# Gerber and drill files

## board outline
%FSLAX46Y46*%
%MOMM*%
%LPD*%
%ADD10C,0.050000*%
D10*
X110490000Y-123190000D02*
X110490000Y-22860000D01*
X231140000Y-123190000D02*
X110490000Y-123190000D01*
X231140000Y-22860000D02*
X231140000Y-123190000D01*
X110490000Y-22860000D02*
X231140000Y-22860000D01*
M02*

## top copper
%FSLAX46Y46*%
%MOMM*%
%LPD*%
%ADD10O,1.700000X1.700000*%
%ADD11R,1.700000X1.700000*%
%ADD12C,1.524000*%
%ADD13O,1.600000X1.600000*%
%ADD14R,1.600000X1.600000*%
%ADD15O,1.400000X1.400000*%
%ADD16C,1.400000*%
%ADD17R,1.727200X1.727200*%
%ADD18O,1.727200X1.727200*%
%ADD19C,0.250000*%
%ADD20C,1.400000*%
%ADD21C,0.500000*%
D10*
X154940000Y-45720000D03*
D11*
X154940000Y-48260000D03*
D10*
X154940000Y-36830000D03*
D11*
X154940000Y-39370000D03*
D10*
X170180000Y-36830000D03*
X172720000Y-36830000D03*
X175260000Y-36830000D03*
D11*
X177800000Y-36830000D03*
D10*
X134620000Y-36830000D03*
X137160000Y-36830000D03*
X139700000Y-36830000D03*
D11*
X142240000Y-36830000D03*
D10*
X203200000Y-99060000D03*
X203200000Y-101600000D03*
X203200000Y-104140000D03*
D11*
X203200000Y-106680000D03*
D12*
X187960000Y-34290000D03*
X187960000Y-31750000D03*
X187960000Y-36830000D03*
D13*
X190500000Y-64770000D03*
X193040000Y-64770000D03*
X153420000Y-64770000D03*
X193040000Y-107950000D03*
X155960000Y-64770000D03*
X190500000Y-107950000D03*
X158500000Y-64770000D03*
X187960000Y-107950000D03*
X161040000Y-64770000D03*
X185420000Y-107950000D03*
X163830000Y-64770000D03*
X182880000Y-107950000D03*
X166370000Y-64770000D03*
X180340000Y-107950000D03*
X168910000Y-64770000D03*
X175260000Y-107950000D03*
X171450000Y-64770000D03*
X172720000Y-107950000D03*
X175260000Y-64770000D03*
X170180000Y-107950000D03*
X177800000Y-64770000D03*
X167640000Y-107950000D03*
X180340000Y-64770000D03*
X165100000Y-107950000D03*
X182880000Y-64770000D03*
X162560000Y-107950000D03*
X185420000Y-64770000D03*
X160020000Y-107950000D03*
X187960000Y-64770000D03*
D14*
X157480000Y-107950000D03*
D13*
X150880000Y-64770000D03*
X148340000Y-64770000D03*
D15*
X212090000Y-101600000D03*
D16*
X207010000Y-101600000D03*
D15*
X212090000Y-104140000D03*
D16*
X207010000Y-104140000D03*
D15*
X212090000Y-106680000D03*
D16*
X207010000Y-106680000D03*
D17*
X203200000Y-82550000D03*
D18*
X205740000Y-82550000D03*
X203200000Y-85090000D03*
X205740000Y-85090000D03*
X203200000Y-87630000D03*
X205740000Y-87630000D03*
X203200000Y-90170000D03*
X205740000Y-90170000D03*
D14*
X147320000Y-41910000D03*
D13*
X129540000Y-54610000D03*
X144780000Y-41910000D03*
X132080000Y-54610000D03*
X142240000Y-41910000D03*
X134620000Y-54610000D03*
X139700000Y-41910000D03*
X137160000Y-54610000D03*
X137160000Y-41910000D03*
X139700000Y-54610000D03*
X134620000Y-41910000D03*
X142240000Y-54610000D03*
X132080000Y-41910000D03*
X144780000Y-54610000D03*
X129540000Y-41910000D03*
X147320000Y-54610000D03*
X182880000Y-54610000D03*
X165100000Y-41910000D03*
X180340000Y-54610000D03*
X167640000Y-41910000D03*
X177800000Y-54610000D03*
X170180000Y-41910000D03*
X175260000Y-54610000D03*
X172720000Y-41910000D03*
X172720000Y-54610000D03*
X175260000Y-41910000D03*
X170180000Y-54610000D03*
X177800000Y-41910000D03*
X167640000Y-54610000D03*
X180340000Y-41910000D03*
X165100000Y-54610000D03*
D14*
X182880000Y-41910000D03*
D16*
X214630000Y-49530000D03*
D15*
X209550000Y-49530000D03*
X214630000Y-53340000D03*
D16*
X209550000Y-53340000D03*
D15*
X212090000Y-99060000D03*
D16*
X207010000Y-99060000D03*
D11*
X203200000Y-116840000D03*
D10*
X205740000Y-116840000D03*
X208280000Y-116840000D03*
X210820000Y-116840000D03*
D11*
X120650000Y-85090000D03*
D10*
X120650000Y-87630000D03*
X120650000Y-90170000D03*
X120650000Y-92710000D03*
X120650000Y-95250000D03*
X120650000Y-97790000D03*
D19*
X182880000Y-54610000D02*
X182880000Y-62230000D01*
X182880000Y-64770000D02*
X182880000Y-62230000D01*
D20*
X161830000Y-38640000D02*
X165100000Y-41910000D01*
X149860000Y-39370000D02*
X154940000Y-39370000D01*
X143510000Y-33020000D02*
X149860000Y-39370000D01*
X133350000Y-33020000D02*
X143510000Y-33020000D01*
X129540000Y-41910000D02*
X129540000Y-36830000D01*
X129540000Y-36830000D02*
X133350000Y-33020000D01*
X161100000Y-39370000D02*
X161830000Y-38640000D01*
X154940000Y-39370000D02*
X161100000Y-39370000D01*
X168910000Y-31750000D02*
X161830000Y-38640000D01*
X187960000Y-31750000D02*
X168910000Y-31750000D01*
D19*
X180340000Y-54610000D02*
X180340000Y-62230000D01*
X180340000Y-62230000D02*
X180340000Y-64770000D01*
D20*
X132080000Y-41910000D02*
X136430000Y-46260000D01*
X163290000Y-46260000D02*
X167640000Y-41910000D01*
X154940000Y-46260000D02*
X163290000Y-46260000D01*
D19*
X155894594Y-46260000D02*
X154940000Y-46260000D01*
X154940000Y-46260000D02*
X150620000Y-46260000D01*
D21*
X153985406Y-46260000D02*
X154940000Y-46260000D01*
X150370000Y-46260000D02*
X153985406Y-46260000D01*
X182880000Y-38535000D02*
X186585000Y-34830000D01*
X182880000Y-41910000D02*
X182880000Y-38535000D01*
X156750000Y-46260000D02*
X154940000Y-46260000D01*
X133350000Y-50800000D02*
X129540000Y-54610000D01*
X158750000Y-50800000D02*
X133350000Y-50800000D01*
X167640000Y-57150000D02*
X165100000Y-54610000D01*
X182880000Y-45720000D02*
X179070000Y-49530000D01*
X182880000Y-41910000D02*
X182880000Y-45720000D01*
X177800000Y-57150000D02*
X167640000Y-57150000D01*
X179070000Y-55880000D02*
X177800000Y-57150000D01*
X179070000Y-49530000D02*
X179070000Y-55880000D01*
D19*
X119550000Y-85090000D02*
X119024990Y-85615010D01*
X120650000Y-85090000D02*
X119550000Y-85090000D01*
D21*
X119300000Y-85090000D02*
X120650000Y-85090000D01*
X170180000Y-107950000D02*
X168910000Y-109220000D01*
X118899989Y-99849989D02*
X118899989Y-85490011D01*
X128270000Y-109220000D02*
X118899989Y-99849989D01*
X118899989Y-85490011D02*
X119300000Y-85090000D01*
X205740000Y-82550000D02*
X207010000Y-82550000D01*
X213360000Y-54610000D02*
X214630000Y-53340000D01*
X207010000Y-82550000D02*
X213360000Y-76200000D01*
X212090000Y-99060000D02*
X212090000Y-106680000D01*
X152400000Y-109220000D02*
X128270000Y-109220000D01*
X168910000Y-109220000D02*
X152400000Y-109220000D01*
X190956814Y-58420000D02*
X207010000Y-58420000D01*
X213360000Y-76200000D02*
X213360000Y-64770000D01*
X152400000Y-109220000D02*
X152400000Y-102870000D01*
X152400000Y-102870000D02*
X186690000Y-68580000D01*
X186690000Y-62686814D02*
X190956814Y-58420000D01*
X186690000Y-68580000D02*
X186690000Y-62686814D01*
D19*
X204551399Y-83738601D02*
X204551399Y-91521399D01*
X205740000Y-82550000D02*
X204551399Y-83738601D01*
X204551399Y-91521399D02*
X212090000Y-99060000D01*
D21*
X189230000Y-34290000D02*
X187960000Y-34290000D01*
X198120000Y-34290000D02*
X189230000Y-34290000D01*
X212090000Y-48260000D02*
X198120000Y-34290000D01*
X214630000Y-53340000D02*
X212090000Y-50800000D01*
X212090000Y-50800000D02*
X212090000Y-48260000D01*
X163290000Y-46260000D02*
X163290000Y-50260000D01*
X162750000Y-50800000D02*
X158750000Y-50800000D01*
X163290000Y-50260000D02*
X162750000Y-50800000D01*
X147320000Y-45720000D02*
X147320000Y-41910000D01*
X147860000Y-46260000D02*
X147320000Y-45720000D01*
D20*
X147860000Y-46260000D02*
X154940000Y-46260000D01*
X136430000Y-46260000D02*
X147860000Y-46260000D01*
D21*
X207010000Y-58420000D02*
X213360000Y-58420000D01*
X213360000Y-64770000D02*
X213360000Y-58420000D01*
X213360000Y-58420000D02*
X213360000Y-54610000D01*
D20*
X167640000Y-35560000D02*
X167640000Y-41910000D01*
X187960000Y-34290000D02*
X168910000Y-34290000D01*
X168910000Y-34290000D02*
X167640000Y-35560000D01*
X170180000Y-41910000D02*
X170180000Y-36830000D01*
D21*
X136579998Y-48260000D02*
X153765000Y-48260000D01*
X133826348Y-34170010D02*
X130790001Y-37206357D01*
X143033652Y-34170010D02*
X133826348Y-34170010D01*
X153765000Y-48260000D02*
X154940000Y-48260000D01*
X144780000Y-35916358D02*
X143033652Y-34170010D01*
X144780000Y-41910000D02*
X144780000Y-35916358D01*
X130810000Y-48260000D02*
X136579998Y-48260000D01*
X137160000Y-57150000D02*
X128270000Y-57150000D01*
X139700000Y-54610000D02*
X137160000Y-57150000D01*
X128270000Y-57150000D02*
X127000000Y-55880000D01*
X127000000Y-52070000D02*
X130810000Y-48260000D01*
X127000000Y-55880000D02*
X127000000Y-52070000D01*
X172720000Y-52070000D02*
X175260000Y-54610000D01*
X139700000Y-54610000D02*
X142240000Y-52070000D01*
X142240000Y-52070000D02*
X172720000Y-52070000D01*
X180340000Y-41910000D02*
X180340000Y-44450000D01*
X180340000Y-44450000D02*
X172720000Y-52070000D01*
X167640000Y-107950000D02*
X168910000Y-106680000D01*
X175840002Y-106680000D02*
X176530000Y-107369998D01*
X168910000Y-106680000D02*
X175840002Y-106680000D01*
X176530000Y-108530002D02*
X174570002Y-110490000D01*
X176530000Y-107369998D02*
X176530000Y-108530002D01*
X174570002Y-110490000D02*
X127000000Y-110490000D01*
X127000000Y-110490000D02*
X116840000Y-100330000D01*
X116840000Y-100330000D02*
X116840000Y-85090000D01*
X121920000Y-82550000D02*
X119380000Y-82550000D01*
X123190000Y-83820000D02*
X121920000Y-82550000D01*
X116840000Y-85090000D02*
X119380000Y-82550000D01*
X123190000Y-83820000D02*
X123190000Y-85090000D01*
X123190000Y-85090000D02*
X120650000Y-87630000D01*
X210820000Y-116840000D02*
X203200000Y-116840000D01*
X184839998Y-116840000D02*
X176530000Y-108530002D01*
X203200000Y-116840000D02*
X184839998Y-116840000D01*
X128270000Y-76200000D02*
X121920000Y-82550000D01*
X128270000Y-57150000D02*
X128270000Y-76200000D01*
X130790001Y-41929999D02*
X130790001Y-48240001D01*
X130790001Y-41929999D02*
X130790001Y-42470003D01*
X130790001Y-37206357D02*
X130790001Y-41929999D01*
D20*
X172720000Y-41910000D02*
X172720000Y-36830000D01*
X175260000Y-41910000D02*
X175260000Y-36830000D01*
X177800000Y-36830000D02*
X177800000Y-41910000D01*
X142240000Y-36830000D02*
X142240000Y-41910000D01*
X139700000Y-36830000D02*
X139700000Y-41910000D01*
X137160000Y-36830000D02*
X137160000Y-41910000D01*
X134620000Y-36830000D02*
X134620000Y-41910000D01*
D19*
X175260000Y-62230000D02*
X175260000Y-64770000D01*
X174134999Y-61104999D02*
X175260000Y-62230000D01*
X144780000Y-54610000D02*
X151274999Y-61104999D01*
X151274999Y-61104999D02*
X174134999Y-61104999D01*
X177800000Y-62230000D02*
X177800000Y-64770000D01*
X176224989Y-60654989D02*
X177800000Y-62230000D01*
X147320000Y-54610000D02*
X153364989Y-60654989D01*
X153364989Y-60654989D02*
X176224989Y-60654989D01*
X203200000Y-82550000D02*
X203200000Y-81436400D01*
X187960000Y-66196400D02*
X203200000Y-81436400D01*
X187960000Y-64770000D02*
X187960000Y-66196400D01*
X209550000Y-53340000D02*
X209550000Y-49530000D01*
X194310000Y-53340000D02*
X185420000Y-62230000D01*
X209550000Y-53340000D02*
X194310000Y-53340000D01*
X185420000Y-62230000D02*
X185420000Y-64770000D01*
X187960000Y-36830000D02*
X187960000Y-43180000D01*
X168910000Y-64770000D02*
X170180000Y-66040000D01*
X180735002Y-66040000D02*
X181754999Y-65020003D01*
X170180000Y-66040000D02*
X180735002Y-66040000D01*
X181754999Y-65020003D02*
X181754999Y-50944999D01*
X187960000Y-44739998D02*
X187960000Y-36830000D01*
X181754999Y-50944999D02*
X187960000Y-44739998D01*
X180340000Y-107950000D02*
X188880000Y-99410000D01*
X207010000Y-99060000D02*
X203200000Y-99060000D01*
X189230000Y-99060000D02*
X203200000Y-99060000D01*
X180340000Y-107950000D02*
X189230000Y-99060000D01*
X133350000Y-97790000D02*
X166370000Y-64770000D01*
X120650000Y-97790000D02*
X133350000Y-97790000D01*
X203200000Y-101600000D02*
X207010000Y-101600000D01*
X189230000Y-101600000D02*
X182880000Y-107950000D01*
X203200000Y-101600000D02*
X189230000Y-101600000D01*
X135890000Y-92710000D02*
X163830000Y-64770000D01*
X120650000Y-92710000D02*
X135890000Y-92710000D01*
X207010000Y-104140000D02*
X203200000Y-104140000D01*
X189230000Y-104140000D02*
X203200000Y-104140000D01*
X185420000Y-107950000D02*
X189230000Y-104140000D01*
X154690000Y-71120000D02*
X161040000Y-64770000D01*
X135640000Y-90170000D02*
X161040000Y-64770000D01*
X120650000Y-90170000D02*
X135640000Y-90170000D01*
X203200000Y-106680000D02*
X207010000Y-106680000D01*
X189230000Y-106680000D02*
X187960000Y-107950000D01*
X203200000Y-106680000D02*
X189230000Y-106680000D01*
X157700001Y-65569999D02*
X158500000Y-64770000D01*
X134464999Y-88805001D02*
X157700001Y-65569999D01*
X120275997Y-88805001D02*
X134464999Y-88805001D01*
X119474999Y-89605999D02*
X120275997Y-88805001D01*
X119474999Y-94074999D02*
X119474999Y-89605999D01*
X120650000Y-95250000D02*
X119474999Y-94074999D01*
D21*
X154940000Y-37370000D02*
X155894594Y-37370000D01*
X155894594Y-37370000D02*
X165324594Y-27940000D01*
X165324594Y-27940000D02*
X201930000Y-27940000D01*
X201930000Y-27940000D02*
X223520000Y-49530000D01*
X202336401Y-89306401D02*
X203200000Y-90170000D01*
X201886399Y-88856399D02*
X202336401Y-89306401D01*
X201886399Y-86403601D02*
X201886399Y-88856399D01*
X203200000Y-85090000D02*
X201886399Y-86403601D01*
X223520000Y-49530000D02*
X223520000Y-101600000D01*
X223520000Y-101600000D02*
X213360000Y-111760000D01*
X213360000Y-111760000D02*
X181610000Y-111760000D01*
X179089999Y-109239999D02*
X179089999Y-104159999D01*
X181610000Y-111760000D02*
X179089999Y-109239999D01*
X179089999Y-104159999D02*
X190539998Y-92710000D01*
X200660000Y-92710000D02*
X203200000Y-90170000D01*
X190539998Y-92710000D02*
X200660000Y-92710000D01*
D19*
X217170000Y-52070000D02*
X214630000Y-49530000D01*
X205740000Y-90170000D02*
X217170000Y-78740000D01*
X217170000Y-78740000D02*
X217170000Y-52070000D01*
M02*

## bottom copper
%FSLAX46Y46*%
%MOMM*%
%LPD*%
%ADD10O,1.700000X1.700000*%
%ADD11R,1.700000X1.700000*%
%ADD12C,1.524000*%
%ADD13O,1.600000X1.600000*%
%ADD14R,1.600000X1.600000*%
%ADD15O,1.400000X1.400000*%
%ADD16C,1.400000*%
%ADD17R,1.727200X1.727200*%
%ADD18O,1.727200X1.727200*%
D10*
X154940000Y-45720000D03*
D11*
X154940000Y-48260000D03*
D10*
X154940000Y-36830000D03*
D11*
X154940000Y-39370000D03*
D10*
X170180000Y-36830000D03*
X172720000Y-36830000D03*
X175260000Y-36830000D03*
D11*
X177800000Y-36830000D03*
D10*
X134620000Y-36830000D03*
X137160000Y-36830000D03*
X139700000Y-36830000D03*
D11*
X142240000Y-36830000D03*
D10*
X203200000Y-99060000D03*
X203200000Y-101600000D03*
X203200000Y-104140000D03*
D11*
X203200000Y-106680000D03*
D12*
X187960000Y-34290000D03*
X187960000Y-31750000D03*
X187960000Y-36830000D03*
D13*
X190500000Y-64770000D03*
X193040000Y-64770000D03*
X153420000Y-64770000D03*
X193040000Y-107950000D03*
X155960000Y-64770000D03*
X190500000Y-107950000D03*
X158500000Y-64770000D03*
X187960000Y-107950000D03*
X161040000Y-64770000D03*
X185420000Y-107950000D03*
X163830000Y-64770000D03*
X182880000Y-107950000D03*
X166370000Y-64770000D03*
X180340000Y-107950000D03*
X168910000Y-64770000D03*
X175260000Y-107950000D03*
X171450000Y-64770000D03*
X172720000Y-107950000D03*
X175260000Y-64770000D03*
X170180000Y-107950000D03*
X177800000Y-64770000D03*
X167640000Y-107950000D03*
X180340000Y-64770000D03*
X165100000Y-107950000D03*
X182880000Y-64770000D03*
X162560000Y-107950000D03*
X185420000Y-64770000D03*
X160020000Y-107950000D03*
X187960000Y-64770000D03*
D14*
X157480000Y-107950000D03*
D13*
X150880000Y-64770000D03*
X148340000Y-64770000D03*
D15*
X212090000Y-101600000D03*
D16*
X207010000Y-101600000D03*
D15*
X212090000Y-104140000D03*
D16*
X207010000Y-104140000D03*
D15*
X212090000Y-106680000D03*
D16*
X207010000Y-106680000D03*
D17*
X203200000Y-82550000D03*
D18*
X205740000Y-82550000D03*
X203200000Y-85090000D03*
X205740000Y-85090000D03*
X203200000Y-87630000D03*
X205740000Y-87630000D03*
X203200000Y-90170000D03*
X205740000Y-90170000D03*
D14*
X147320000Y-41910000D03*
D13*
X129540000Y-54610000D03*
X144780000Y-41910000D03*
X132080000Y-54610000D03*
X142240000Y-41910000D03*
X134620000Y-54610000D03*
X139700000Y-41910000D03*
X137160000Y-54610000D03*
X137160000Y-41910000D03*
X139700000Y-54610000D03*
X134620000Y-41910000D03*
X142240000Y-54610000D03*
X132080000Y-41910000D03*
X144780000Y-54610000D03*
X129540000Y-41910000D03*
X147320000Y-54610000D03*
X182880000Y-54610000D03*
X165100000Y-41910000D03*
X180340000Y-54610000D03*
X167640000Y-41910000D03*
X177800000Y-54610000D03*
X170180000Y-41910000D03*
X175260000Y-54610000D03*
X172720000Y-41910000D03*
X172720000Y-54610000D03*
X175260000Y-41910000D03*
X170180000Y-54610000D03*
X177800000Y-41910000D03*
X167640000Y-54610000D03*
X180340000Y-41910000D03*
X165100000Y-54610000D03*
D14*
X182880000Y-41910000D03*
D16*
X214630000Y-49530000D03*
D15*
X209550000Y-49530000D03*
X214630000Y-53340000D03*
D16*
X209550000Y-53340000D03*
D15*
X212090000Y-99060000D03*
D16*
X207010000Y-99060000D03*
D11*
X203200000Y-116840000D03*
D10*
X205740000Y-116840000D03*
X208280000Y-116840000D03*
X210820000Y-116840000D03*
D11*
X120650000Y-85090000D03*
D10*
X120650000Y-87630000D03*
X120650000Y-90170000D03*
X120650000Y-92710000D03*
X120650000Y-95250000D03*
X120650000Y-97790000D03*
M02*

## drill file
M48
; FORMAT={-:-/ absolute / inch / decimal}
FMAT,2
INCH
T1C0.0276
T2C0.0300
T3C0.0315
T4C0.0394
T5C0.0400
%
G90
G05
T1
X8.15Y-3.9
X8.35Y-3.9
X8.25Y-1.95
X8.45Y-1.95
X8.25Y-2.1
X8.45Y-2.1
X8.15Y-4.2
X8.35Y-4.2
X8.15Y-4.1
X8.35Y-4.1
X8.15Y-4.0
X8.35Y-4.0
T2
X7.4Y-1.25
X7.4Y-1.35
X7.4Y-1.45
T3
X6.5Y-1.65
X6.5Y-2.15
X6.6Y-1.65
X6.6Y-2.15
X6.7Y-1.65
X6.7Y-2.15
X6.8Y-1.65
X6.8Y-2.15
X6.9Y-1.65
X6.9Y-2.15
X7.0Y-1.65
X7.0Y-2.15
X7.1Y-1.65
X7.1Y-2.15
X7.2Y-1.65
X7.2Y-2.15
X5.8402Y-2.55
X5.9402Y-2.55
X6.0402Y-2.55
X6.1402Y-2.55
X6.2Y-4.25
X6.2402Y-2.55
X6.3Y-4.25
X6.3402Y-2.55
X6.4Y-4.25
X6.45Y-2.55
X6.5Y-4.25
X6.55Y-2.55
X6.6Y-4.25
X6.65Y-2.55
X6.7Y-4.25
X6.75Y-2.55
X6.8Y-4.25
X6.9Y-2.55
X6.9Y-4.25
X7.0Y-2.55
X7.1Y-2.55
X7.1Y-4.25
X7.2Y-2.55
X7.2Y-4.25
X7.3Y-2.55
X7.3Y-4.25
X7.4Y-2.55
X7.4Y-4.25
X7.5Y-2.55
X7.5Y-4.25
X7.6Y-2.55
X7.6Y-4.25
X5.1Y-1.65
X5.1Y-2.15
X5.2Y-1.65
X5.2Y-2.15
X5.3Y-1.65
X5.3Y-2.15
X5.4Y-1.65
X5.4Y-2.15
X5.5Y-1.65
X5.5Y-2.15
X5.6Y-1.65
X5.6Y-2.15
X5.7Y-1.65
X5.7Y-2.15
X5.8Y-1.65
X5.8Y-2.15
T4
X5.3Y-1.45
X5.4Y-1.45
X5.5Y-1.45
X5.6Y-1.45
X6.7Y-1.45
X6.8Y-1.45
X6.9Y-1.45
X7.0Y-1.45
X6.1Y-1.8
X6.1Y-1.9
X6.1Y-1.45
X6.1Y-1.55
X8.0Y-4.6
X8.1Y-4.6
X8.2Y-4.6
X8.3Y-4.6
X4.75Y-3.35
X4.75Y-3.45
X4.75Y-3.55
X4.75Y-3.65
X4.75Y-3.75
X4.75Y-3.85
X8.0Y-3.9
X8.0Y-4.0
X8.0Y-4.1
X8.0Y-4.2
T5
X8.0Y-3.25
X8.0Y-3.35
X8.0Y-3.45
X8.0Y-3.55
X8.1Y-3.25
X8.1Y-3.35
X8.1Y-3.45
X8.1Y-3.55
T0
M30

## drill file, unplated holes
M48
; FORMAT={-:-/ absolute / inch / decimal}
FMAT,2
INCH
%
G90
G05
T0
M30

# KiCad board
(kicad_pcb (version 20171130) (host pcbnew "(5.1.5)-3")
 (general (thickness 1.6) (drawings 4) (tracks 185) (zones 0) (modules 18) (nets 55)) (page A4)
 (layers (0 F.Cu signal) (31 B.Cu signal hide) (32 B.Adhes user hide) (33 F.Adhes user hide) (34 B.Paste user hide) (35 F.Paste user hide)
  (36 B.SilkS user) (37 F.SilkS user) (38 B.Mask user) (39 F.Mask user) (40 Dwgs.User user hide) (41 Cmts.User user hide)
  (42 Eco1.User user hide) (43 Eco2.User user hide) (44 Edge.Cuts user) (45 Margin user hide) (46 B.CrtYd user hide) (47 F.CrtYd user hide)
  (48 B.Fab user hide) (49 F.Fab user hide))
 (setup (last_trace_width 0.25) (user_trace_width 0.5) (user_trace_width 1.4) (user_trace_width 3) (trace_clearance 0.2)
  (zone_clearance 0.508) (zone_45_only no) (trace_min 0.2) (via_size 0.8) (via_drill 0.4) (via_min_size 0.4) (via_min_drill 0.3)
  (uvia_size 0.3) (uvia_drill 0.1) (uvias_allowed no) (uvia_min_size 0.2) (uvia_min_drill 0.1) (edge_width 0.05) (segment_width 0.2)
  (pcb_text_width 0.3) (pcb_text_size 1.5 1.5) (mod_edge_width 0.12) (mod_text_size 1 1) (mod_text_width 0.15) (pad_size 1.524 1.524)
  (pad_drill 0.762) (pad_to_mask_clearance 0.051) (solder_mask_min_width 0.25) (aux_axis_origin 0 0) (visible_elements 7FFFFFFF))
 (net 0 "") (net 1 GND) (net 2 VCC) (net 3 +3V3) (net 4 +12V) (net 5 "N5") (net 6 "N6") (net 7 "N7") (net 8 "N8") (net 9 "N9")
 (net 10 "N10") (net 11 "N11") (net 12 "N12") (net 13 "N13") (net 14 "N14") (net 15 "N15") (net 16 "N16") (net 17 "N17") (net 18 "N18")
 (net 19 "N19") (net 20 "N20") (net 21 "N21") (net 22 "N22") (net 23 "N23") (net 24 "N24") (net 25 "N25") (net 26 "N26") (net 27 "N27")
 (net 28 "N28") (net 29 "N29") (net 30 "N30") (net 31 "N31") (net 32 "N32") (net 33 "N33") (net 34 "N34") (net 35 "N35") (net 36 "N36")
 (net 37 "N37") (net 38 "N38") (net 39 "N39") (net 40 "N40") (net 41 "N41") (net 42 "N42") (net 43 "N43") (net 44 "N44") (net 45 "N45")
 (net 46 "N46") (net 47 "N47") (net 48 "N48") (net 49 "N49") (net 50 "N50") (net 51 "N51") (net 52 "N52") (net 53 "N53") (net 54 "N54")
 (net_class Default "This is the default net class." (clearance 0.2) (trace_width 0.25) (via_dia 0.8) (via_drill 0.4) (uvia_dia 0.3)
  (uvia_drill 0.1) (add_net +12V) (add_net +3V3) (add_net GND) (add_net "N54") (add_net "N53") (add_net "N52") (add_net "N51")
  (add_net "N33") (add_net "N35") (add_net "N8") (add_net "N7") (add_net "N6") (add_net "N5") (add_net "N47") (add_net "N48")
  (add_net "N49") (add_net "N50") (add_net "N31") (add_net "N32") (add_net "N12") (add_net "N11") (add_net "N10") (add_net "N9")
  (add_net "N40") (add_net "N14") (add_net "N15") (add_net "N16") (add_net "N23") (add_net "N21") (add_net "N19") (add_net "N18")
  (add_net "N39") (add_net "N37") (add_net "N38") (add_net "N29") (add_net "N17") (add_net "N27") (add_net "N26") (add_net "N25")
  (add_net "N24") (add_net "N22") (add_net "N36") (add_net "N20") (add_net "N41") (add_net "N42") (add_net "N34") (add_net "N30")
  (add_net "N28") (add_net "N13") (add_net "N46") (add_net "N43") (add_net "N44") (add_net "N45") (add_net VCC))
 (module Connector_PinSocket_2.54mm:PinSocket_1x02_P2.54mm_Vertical (layer F.Cu) (at 154.94 48.26 180)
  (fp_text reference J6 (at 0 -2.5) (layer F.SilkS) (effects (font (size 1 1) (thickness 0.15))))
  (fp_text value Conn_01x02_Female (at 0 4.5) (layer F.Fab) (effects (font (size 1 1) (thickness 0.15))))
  (pad 2 thru_hole oval (at 0 2.54 180) (size 1.7 1.7) (drill 1) (layers *.Cu *.Mask) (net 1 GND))
  (pad 1 thru_hole rect (at 0 0 180) (size 1.7 1.7) (drill 1) (layers *.Cu *.Mask) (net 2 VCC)))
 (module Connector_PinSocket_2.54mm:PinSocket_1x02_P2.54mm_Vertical (layer F.Cu) (at 154.94 39.37 180)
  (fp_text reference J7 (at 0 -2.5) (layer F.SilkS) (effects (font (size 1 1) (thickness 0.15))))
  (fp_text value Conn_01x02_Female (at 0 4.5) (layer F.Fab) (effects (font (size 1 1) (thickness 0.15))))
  (pad 2 thru_hole oval (at 0 2.54 180) (size 1.7 1.7) (drill 1) (layers *.Cu *.Mask) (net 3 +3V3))
  (pad 1 thru_hole rect (at 0 0 180) (size 1.7 1.7) (drill 1) (layers *.Cu *.Mask) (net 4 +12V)))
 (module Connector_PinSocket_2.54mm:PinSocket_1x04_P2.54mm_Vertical (layer F.Cu) (at 177.8 36.83 270)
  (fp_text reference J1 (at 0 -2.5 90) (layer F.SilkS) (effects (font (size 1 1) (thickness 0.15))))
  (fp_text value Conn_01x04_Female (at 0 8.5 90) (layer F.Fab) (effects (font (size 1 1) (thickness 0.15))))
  (pad 4 thru_hole oval (at 0 7.62 270) (size 1.7 1.7) (drill 1) (layers *.Cu *.Mask) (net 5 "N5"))
  (pad 3 thru_hole oval (at 0 5.08 270) (size 1.7 1.7) (drill 1) (layers *.Cu *.Mask) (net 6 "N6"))
  (pad 2 thru_hole oval (at 0 2.54 270) (size 1.7 1.7) (drill 1) (layers *.Cu *.Mask) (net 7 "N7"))
  (pad 1 thru_hole rect (at 0 0 270) (size 1.7 1.7) (drill 1) (layers *.Cu *.Mask) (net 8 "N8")))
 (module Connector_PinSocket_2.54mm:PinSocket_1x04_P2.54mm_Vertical (layer F.Cu) (at 142.24 36.83 270)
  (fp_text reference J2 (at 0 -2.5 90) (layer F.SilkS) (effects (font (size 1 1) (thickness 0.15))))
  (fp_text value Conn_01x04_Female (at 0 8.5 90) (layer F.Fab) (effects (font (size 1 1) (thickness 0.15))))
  (pad 4 thru_hole oval (at 0 7.62 270) (size 1.7 1.7) (drill 1) (layers *.Cu *.Mask) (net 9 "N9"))
  (pad 3 thru_hole oval (at 0 5.08 270) (size 1.7 1.7) (drill 1) (layers *.Cu *.Mask) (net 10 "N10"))
  (pad 2 thru_hole oval (at 0 2.54 270) (size 1.7 1.7) (drill 1) (layers *.Cu *.Mask) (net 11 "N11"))
  (pad 1 thru_hole rect (at 0 0 270) (size 1.7 1.7) (drill 1) (layers *.Cu *.Mask) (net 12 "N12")))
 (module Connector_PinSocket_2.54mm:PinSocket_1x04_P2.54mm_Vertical (layer F.Cu) (at 203.2 106.68 180)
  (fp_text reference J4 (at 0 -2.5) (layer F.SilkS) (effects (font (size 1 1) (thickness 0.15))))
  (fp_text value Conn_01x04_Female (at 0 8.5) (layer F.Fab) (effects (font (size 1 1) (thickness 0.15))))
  (pad 4 thru_hole oval (at 0 7.62 180) (size 1.7 1.7) (drill 1) (layers *.Cu *.Mask) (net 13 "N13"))
  (pad 3 thru_hole oval (at 0 5.08 180) (size 1.7 1.7) (drill 1) (layers *.Cu *.Mask) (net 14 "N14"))
  (pad 2 thru_hole oval (at 0 2.54 180) (size 1.7 1.7) (drill 1) (layers *.Cu *.Mask) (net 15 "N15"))
  (pad 1 thru_hole rect (at 0 0 180) (size 1.7 1.7) (drill 1) (layers *.Cu *.Mask) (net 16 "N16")))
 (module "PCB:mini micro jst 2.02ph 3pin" (layer F.Cu) (at 194.31 33.02 90)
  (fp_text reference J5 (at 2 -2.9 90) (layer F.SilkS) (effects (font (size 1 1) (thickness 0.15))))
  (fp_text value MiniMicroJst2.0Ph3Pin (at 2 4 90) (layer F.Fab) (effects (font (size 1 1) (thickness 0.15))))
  (pad 2 thru_hole circle (at -1.27 -6.35 90) (size 1.524 1.524) (drill 0.762) (layers *.Cu *.Mask) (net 1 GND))
  (pad 3 thru_hole circle (at 1.27 -6.35 90) (size 1.524 1.524) (drill 0.762) (layers *.Cu *.Mask) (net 4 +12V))
  (pad 1 thru_hole circle (at -3.81 -6.35 90) (size 1.524 1.524) (drill 0.762) (layers *.Cu *.Mask) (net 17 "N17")))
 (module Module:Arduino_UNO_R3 (layer B.Cu) (at 157.48 110.49)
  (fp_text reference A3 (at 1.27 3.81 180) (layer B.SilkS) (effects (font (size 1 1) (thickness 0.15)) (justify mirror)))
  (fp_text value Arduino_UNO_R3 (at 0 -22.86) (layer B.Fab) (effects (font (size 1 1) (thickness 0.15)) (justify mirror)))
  (pad 16 thru_hole oval (at 33.02 -45.72 270) (size 1.6 1.6) (drill 0.8) (layers *.Cu *.Mask) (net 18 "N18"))
  (pad 15 thru_hole oval (at 35.56 -45.72 270) (size 1.6 1.6) (drill 0.8) (layers *.Cu *.Mask) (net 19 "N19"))
  (pad 30 thru_hole oval (at -4.06 -45.72 270) (size 1.6 1.6) (drill 0.8) (layers *.Cu *.Mask) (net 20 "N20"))
  (pad 14 thru_hole oval (at 35.56 -2.54 270) (size 1.6 1.6) (drill 0.8) (layers *.Cu *.Mask) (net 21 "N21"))
  (pad 29 thru_hole oval (at -1.52 -45.72 270) (size 1.6 1.6) (drill 0.8) (layers *.Cu *.Mask) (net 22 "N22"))
  (pad 13 thru_hole oval (at 33.02 -2.54 270) (size 1.6 1.6) (drill 0.8) (layers *.Cu *.Mask) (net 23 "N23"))
  (pad 28 thru_hole oval (at 1.02 -45.72 270) (size 1.6 1.6) (drill 0.8) (layers *.Cu *.Mask) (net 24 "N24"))
  (pad 12 thru_hole oval (at 30.48 -2.54 270) (size 1.6 1.6) (drill 0.8) (layers *.Cu *.Mask) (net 16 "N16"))
  (pad 27 thru_hole oval (at 3.56 -45.72 270) (size 1.6 1.6) (drill 0.8) (layers *.Cu *.Mask) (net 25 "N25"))
  (pad 11 thru_hole oval (at 27.94 -2.54 270) (size 1.6 1.6) (drill 0.8) (layers *.Cu *.Mask) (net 15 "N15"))
  (pad 26 thru_hole oval (at 6.35 -45.72 270) (size 1.6 1.6) (drill 0.8) (layers *.Cu *.Mask) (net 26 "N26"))
  (pad 10 thru_hole oval (at 25.4 -2.54 270) (size 1.6 1.6) (drill 0.8) (layers *.Cu *.Mask) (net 14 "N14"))
  (pad 25 thru_hole oval (at 8.89 -45.72 270) (size 1.6 1.6) (drill 0.8) (layers *.Cu *.Mask) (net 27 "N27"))
  (pad 9 thru_hole oval (at 22.86 -2.54 270) (size 1.6 1.6) (drill 0.8) (layers *.Cu *.Mask) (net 13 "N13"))
  (pad 24 thru_hole oval (at 11.43 -45.72 270) (size 1.6 1.6) (drill 0.8) (layers *.Cu *.Mask) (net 17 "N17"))
  (pad 8 thru_hole oval (at 17.78 -2.54 270) (size 1.6 1.6) (drill 0.8) (layers *.Cu *.Mask) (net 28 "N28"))
  (pad 23 thru_hole oval (at 13.97 -45.72 270) (size 1.6 1.6) (drill 0.8) (layers *.Cu *.Mask) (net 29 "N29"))
  (pad 7 thru_hole oval (at 15.24 -2.54 270) (size 1.6 1.6) (drill 0.8) (layers *.Cu *.Mask) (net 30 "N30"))
  (pad 22 thru_hole oval (at 17.78 -45.72 270) (size 1.6 1.6) (drill 0.8) (layers *.Cu *.Mask) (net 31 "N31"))
  (pad 6 thru_hole oval (at 12.7 -2.54 270) (size 1.6 1.6) (drill 0.8) (layers *.Cu *.Mask) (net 1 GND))
  (pad 21 thru_hole oval (at 20.32 -45.72 270) (size 1.6 1.6) (drill 0.8) (layers *.Cu *.Mask) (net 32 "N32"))
  (pad 5 thru_hole oval (at 10.16 -2.54 270) (size 1.6 1.6) (drill 0.8) (layers *.Cu *.Mask) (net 2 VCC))
  (pad 20 thru_hole oval (at 22.86 -45.72 270) (size 1.6 1.6) (drill 0.8) (layers *.Cu *.Mask) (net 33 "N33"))
  (pad 4 thru_hole oval (at 7.62 -2.54 270) (size 1.6 1.6) (drill 0.8) (layers *.Cu *.Mask) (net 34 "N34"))
  (pad 19 thru_hole oval (at 25.4 -45.72 270) (size 1.6 1.6) (drill 0.8) (layers *.Cu *.Mask) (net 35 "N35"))
  (pad 3 thru_hole oval (at 5.08 -2.54 270) (size 1.6 1.6) (drill 0.8) (layers *.Cu *.Mask) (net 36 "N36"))
  (pad 18 thru_hole oval (at 27.94 -45.72 270) (size 1.6 1.6) (drill 0.8) (layers *.Cu *.Mask) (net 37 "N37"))
  (pad 2 thru_hole oval (at 2.54 -2.54 270) (size 1.6 1.6) (drill 0.8) (layers *.Cu *.Mask) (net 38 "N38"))
  (pad 17 thru_hole oval (at 30.48 -45.72 270) (size 1.6 1.6) (drill 0.8) (layers *.Cu *.Mask) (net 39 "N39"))
  (pad 1 thru_hole rect (at 0 -2.54 270) (size 1.6 1.6) (drill 0.8) (layers *.Cu *.Mask) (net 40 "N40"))
  (pad 31 thru_hole oval (at -6.6 -45.72 270) (size 1.6 1.6) (drill 0.8) (layers *.Cu *.Mask) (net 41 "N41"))
  (pad 32 thru_hole oval (at -9.14 -45.72 270) (size 1.6 1.6) (drill 0.8) (layers *.Cu *.Mask) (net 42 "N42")))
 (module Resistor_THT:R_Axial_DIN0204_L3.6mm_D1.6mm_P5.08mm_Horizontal (layer F.Cu) (at 207.01 101.6)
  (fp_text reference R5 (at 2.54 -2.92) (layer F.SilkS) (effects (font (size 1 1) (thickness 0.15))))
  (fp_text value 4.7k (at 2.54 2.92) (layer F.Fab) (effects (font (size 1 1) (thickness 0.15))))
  (pad 2 thru_hole oval (at 5.08 0) (size 1.4 1.4) (drill 0.7) (layers *.Cu *.Mask) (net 1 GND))
  (pad 1 thru_hole circle (at 0 0) (size 1.4 1.4) (drill 0.7) (layers *.Cu *.Mask) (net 14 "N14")))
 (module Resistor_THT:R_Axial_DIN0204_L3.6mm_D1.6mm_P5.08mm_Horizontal (layer F.Cu) (at 207.01 104.14)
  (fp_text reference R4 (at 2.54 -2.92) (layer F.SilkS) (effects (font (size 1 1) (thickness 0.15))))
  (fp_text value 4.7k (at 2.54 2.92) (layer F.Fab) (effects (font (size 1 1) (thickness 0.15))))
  (pad 2 thru_hole oval (at 5.08 0) (size 1.4 1.4) (drill 0.7) (layers *.Cu *.Mask) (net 1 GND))
  (pad 1 thru_hole circle (at 0 0) (size 1.4 1.4) (drill 0.7) (layers *.Cu *.Mask) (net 15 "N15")))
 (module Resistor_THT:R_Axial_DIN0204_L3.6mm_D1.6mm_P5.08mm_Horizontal (layer F.Cu) (at 207.01 106.68)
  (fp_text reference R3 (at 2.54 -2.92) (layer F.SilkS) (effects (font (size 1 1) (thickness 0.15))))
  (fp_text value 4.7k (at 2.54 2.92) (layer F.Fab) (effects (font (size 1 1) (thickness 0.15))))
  (pad 2 thru_hole oval (at 5.08 0) (size 1.4 1.4) (drill 0.7) (layers *.Cu *.Mask) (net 1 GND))
  (pad 1 thru_hole circle (at 0 0) (size 1.4 1.4) (drill 0.7) (layers *.Cu *.Mask) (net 16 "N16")))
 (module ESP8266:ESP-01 (layer F.Cu) (at 203.2 82.55)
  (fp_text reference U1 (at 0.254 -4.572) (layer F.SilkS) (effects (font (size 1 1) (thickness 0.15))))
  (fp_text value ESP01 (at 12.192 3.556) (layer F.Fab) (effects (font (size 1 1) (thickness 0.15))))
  (pad 1 thru_hole rect (at 0 0) (size 1.7272 1.7272) (drill 1.016) (layers *.Cu *.Mask F.SilkS) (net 39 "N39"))
  (pad 2 thru_hole oval (at 2.54 0) (size 1.7272 1.7272) (drill 1.016) (layers *.Cu *.Mask F.SilkS) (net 1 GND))
  (pad 3 thru_hole oval (at 0 2.54) (size 1.7272 1.7272) (drill 1.016) (layers *.Cu *.Mask F.SilkS) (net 3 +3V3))
  (pad 4 thru_hole oval (at 2.54 2.54) (size 1.7272 1.7272) (drill 1.016) (layers *.Cu *.Mask F.SilkS) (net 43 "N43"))
  (pad 5 thru_hole oval (at 0 5.08) (size 1.7272 1.7272) (drill 1.016) (layers *.Cu *.Mask F.SilkS) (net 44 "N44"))
  (pad 6 thru_hole oval (at 2.54 5.08) (size 1.7272 1.7272) (drill 1.016) (layers *.Cu *.Mask F.SilkS) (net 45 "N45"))
  (pad 7 thru_hole oval (at 0 7.62) (size 1.7272 1.7272) (drill 1.016) (layers *.Cu *.Mask F.SilkS) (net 3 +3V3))
  (pad 8 thru_hole oval (at 2.54 7.62) (size 1.7272 1.7272) (drill 1.016) (layers *.Cu *.Mask F.SilkS) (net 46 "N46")))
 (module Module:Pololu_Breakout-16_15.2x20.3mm (layer F.Cu) (at 147.32 41.91 270)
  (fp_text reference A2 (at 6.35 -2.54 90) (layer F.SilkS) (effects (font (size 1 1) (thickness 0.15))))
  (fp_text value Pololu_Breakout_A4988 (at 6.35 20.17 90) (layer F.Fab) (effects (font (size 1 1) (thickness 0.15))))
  (pad 1 thru_hole rect (at 0 0 270) (size 1.6 1.6) (drill 0.8) (layers *.Cu *.Mask) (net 1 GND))
  (pad 9 thru_hole oval (at 12.7 17.78 270) (size 1.6 1.6) (drill 0.8) (layers *.Cu *.Mask) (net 1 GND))
  (pad 2 thru_hole oval (at 0 2.54 270) (size 1.6 1.6) (drill 0.8) (layers *.Cu *.Mask) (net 2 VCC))
  (pad 10 thru_hole oval (at 12.7 15.24 270) (size 1.6 1.6) (drill 0.8) (layers *.Cu *.Mask) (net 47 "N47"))
  (pad 3 thru_hole oval (at 0 5.08 270) (size 1.6 1.6) (drill 0.8) (layers *.Cu *.Mask) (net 12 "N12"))
  (pad 11 thru_hole oval (at 12.7 12.7 270) (size 1.6 1.6) (drill 0.8) (layers *.Cu *.Mask) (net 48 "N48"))
  (pad 4 thru_hole oval (at 0 7.62 270) (size 1.6 1.6) (drill 0.8) (layers *.Cu *.Mask) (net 11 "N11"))
  (pad 12 thru_hole oval (at 12.7 10.16 270) (size 1.6 1.6) (drill 0.8) (layers *.Cu *.Mask) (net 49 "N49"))
  (pad 5 thru_hole oval (at 0 10.16 270) (size 1.6 1.6) (drill 0.8) (layers *.Cu *.Mask) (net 10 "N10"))
  (pad 13 thru_hole oval (at 12.7 7.62 270) (size 1.6 1.6) (drill 0.8) (layers *.Cu *.Mask) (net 2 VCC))
  (pad 6 thru_hole oval (at 0 12.7 270) (size 1.6 1.6) (drill 0.8) (layers *.Cu *.Mask) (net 9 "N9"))
  (pad 14 thru_hole oval (at 12.7 5.08 270) (size 1.6 1.6) (drill 0.8) (layers *.Cu *.Mask) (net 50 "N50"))
  (pad 7 thru_hole oval (at 0 15.24 270) (size 1.6 1.6) (drill 0.8) (layers *.Cu *.Mask) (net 1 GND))
  (pad 15 thru_hole oval (at 12.7 2.54 270) (size 1.6 1.6) (drill 0.8) (layers *.Cu *.Mask) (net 31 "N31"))
  (pad 8 thru_hole oval (at 0 17.78 270) (size 1.6 1.6) (drill 0.8) (layers *.Cu *.Mask) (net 4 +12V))
  (pad 16 thru_hole oval (at 12.7 0 270) (size 1.6 1.6) (drill 0.8) (layers *.Cu *.Mask) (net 32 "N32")))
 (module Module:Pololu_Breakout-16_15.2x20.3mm (layer F.Cu) (at 182.88 41.91 270)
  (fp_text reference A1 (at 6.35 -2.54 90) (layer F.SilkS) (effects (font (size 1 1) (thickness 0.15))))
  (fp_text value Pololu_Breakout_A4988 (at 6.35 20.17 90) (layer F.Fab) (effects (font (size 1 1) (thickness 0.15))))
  (pad 16 thru_hole oval (at 12.7 0 270) (size 1.6 1.6) (drill 0.8) (layers *.Cu *.Mask) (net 35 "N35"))
  (pad 8 thru_hole oval (at 0 17.78 270) (size 1.6 1.6) (drill 0.8) (layers *.Cu *.Mask) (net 4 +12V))
  (pad 15 thru_hole oval (at 12.7 2.54 270) (size 1.6 1.6) (drill 0.8) (layers *.Cu *.Mask) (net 33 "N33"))
  (pad 7 thru_hole oval (at 0 15.24 270) (size 1.6 1.6) (drill 0.8) (layers *.Cu *.Mask) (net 1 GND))
  (pad 14 thru_hole oval (at 12.7 5.08 270) (size 1.6 1.6) (drill 0.8) (layers *.Cu *.Mask) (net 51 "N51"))
  (pad 6 thru_hole oval (at 0 12.7 270) (size 1.6 1.6) (drill 0.8) (layers *.Cu *.Mask) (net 5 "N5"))
  (pad 13 thru_hole oval (at 12.7 7.62 270) (size 1.6 1.6) (drill 0.8) (layers *.Cu *.Mask) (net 2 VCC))
  (pad 5 thru_hole oval (at 0 10.16 270) (size 1.6 1.6) (drill 0.8) (layers *.Cu *.Mask) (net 6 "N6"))
  (pad 12 thru_hole oval (at 12.7 10.16 270) (size 1.6 1.6) (drill 0.8) (layers *.Cu *.Mask) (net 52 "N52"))
  (pad 4 thru_hole oval (at 0 7.62 270) (size 1.6 1.6) (drill 0.8) (layers *.Cu *.Mask) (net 7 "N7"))
  (pad 11 thru_hole oval (at 12.7 12.7 270) (size 1.6 1.6) (drill 0.8) (layers *.Cu *.Mask) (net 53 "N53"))
  (pad 3 thru_hole oval (at 0 5.08 270) (size 1.6 1.6) (drill 0.8) (layers *.Cu *.Mask) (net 8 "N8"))
  (pad 10 thru_hole oval (at 12.7 15.24 270) (size 1.6 1.6) (drill 0.8) (layers *.Cu *.Mask) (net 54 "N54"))
  (pad 2 thru_hole oval (at 0 2.54 270) (size 1.6 1.6) (drill 0.8) (layers *.Cu *.Mask) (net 2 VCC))
  (pad 9 thru_hole oval (at 12.7 17.78 270) (size 1.6 1.6) (drill 0.8) (layers *.Cu *.Mask) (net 1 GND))
  (pad 1 thru_hole rect (at 0 0 270) (size 1.6 1.6) (drill 0.8) (layers *.Cu *.Mask) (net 1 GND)))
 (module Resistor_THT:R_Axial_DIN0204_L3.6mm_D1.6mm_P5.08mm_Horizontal (layer F.Cu) (at 214.63 49.53 180)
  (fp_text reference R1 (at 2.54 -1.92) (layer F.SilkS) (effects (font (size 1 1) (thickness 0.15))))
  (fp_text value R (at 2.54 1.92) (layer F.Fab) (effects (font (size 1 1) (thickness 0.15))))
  (pad 1 thru_hole circle (at 0 0 180) (size 1.4 1.4) (drill 0.7) (layers *.Cu *.Mask) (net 46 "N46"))
  (pad 2 thru_hole oval (at 5.08 0 180) (size 1.4 1.4) (drill 0.7) (layers *.Cu *.Mask) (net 37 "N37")))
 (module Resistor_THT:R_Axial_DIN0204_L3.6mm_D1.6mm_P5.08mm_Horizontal (layer F.Cu) (at 209.55 53.34)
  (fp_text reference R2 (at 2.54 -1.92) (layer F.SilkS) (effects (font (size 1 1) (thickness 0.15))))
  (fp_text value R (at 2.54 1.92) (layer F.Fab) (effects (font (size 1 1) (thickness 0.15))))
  (pad 2 thru_hole oval (at 5.08 0) (size 1.4 1.4) (drill 0.7) (layers *.Cu *.Mask) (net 1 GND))
  (pad 1 thru_hole circle (at 0 0) (size 1.4 1.4) (drill 0.7) (layers *.Cu *.Mask) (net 37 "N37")))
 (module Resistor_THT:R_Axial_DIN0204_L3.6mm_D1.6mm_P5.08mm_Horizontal (layer F.Cu) (at 207.01 99.06)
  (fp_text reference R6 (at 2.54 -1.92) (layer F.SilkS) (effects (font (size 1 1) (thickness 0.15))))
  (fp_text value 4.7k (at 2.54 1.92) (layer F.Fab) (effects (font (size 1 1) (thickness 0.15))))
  (pad 2 thru_hole oval (at 5.08 0) (size 1.4 1.4) (drill 0.7) (layers *.Cu *.Mask) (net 1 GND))
  (pad 1 thru_hole circle (at 0 0) (size 1.4 1.4) (drill 0.7) (layers *.Cu *.Mask) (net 13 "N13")))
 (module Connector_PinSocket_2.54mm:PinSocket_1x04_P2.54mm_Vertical (layer F.Cu) (at 203.2 116.84 90)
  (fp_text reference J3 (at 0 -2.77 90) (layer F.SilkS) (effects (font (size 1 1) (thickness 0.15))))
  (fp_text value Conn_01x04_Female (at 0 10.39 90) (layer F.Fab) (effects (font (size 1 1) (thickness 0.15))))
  (pad 1 thru_hole rect (at 0 0 90) (size 1.7 1.7) (drill 1) (layers *.Cu *.Mask) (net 2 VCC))
  (pad 2 thru_hole oval (at 0 2.54 90) (size 1.7 1.7) (drill 1) (layers *.Cu *.Mask) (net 2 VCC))
  (pad 3 thru_hole oval (at 0 5.08 90) (size 1.7 1.7) (drill 1) (layers *.Cu *.Mask) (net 2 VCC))
  (pad 4 thru_hole oval (at 0 7.62 90) (size 1.7 1.7) (drill 1) (layers *.Cu *.Mask) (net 2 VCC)))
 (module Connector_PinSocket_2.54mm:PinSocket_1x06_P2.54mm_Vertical (layer F.Cu) (at 120.65 85.09)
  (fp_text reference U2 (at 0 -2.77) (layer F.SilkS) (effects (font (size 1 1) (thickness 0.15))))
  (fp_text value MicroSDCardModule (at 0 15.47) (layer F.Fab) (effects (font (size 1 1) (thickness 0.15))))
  (pad 1 thru_hole rect (at 0 0) (size 1.7 1.7) (drill 1) (layers *.Cu *.Mask) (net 1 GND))
  (pad 2 thru_hole oval (at 0 2.54) (size 1.7 1.7) (drill 1) (layers *.Cu *.Mask) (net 2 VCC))
  (pad 3 thru_hole oval (at 0 5.08) (size 1.7 1.7) (drill 1) (layers *.Cu *.Mask) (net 25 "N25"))
  (pad 4 thru_hole oval (at 0 7.62) (size 1.7 1.7) (drill 1) (layers *.Cu *.Mask) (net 26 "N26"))
  (pad 5 thru_hole oval (at 0 10.16) (size 1.7 1.7) (drill 1) (layers *.Cu *.Mask) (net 24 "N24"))
  (pad 6 thru_hole oval (at 0 12.7) (size 1.7 1.7) (drill 1) (layers *.Cu *.Mask) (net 27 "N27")))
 (gr_line (start 110.49 123.19) (end 110.49 22.86) (layer Edge.Cuts) (width 0.05))
 (gr_line (start 231.14 123.19) (end 110.49 123.19) (layer Edge.Cuts) (width 0.05))
 (gr_line (start 231.14 22.86) (end 231.14 123.19) (layer Edge.Cuts) (width 0.05))
 (gr_line (start 110.49 22.86) (end 231.14 22.86) (layer Edge.Cuts) (width 0.05))
 (segment (start 182.88 54.61) (end 182.88 62.23) (width 0.25) (layer F.Cu) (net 35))
 (segment (start 182.88 64.77) (end 182.88 62.23) (width 0.25) (layer F.Cu) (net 35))
 (segment (start 161.83 38.64) (end 165.1 41.91) (width 1.4) (layer F.Cu) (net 4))
 (segment (start 149.86 39.37) (end 154.94 39.37) (width 1.4) (layer F.Cu) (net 4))
 (segment (start 143.51 33.02) (end 149.86 39.37) (width 1.4) (layer F.Cu) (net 4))
 (segment (start 133.35 33.02) (end 143.51 33.02) (width 1.4) (layer F.Cu) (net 4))
 (segment (start 129.54 41.91) (end 129.54 36.83) (width 1.4) (layer F.Cu) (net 4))
 (segment (start 129.54 36.83) (end 133.35 33.02) (width 1.4) (layer F.Cu) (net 4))
 (segment (start 161.1 39.37) (end 161.83 38.64) (width 1.4) (layer F.Cu) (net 4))
 (segment (start 154.94 39.37) (end 161.1 39.37) (width 1.4) (layer F.Cu) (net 4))
 (segment (start 168.91 31.75) (end 161.83 38.64) (width 1.4) (layer F.Cu) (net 4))
 (segment (start 187.96 31.75) (end 168.91 31.75) (width 1.4) (layer F.Cu) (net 4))
 (segment (start 180.34 54.61) (end 180.34 62.23) (width 0.25) (layer F.Cu) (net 33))
 (segment (start 180.34 62.23) (end 180.34 64.77) (width 0.25) (layer F.Cu) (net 33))
 (segment (start 132.08 41.91) (end 136.43 46.26) (width 1.4) (layer F.Cu) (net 1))
 (segment (start 163.29 46.26) (end 167.64 41.91) (width 1.4) (layer F.Cu) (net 1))
 (segment (start 154.94 46.26) (end 163.29 46.26) (width 1.4) (layer F.Cu) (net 1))
 (segment (start 155.894594 46.26) (end 154.94 46.26) (width 0.25) (layer F.Cu) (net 1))
 (segment (start 154.94 46.26) (end 150.62 46.26) (width 0.25) (layer F.Cu) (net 1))
 (segment (start 153.985406 46.26) (end 154.94 46.26) (width 0.5) (layer F.Cu) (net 1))
 (segment (start 150.37 46.26) (end 153.985406 46.26) (width 0.5) (layer F.Cu) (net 1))
 (segment (start 182.88 38.535) (end 186.585 34.83) (width 0.5) (layer F.Cu) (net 1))
 (segment (start 182.88 41.91) (end 182.88 38.535) (width 0.5) (layer F.Cu) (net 1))
 (segment (start 156.75 46.26) (end 154.94 46.26) (width 0.5) (layer F.Cu) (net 1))
 (segment (start 133.35 50.8) (end 129.54 54.61) (width 0.5) (layer F.Cu) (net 1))
 (segment (start 158.75 50.8) (end 133.35 50.8) (width 0.5) (layer F.Cu) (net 1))
 (segment (start 167.64 57.15) (end 165.1 54.61) (width 0.5) (layer F.Cu) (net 1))
 (segment (start 182.88 45.72) (end 179.07 49.53) (width 0.5) (layer F.Cu) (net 1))
 (segment (start 182.88 41.91) (end 182.88 45.72) (width 0.5) (layer F.Cu) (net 1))
 (segment (start 177.8 57.15) (end 167.64 57.15) (width 0.5) (layer F.Cu) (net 1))
 (segment (start 179.07 55.88) (end 177.8 57.15) (width 0.5) (layer F.Cu) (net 1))
 (segment (start 179.07 49.53) (end 179.07 55.88) (width 0.5) (layer F.Cu) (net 1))
 (segment (start 119.55 85.09) (end 119.02499 85.61501) (width 0.25) (layer F.Cu) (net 1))
 (segment (start 120.65 85.09) (end 119.55 85.09) (width 0.25) (layer F.Cu) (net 1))
 (segment (start 119.3 85.09) (end 120.65 85.09) (width 0.5) (layer F.Cu) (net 1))
 (segment (start 170.18 107.95) (end 168.91 109.22) (width 0.5) (layer F.Cu) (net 1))
 (segment (start 118.899989 99.849989) (end 118.899989 85.490011) (width 0.5) (layer F.Cu) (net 1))
 (segment (start 128.27 109.22) (end 118.899989 99.849989) (width 0.5) (layer F.Cu) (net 1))
 (segment (start 118.899989 85.490011) (end 119.3 85.09) (width 0.5) (layer F.Cu) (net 1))
 (segment (start 205.74 82.55) (end 207.01 82.55) (width 0.5) (layer F.Cu) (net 1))
 (segment (start 213.36 54.61) (end 214.63 53.34) (width 0.5) (layer F.Cu) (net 1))
 (segment (start 207.01 82.55) (end 213.36 76.2) (width 0.5) (layer F.Cu) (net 1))
 (segment (start 212.09 99.06) (end 212.09 106.68) (width 0.5) (layer F.Cu) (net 1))
 (segment (start 152.4 109.22) (end 128.27 109.22) (width 0.5) (layer F.Cu) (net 1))
 (segment (start 168.91 109.22) (end 152.4 109.22) (width 0.5) (layer F.Cu) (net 1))
 (segment (start 190.956814 58.42) (end 207.01 58.42) (width 0.5) (layer F.Cu) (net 1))
 (segment (start 213.36 76.2) (end 213.36 64.77) (width 0.5) (layer F.Cu) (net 1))
 (segment (start 152.4 109.22) (end 152.4 102.87) (width 0.5) (layer F.Cu) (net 1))
 (segment (start 152.4 102.87) (end 186.69 68.58) (width 0.5) (layer F.Cu) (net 1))
 (segment (start 186.69 62.686814) (end 190.956814 58.42) (width 0.5) (layer F.Cu) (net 1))
 (segment (start 186.69 68.58) (end 186.69 62.686814) (width 0.5) (layer F.Cu) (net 1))
 (segment (start 204.551399 83.738601) (end 204.551399 91.521399) (width 0.25) (layer F.Cu) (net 1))
 (segment (start 205.74 82.55) (end 204.551399 83.738601) (width 0.25) (layer F.Cu) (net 1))
 (segment (start 204.551399 91.521399) (end 212.09 99.06) (width 0.25) (layer F.Cu) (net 1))
 (segment (start 189.23 34.29) (end 187.96 34.29) (width 0.5) (layer F.Cu) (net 1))
 (segment (start 198.12 34.29) (end 189.23 34.29) (width 0.5) (layer F.Cu) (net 1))
 (segment (start 212.09 48.26) (end 198.12 34.29) (width 0.5) (layer F.Cu) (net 1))
 (segment (start 214.63 53.34) (end 212.09 50.8) (width 0.5) (layer F.Cu) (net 1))
 (segment (start 212.09 50.8) (end 212.09 48.26) (width 0.5) (layer F.Cu) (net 1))
 (segment (start 163.29 46.26) (end 163.29 50.26) (width 0.5) (layer F.Cu) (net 1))
 (segment (start 162.75 50.8) (end 158.75 50.8) (width 0.5) (layer F.Cu) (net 1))
 (segment (start 163.29 50.26) (end 162.75 50.8) (width 0.5) (layer F.Cu) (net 1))
 (segment (start 147.32 45.72) (end 147.32 41.91) (width 0.5) (layer F.Cu) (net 1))
 (segment (start 147.86 46.26) (end 147.32 45.72) (width 0.5) (layer F.Cu) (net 1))
 (segment (start 147.86 46.26) (end 154.94 46.26) (width 1.4) (layer F.Cu) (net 1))
 (segment (start 136.43 46.26) (end 147.86 46.26) (width 1.4) (layer F.Cu) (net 1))
 (segment (start 207.01 58.42) (end 213.36 58.42) (width 0.5) (layer F.Cu) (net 1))
 (segment (start 213.36 64.77) (end 213.36 58.42) (width 0.5) (layer F.Cu) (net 1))
 (segment (start 213.36 58.42) (end 213.36 54.61) (width 0.5) (layer F.Cu) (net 1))
 (segment (start 167.64 35.56) (end 167.64 41.91) (width 1.4) (layer F.Cu) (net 1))
 (segment (start 187.96 34.29) (end 168.91 34.29) (width 1.4) (layer F.Cu) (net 1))
 (segment (start 168.91 34.29) (end 167.64 35.56) (width 1.4) (layer F.Cu) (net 1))
 (segment (start 170.18 41.91) (end 170.18 36.83) (width 1.4) (layer F.Cu) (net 5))
 (segment (start 136.579998 48.26) (end 153.765 48.26) (width 0.5) (layer F.Cu) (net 2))
 (segment (start 133.826348 34.17001) (end 130.790001 37.206357) (width 0.5) (layer F.Cu) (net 2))
 (segment (start 143.033652 34.17001) (end 133.826348 34.17001) (width 0.5) (layer F.Cu) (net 2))
 (segment (start 153.765 48.26) (end 154.94 48.26) (width 0.5) (layer F.Cu) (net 2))
 (segment (start 144.78 35.916358) (end 143.033652 34.17001) (width 0.5) (layer F.Cu) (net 2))
 (segment (start 144.78 41.91) (end 144.78 35.916358) (width 0.5) (layer F.Cu) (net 2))
 (segment (start 130.81 48.26) (end 136.579998 48.26) (width 0.5) (layer F.Cu) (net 2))
 (segment (start 137.16 57.15) (end 128.27 57.15) (width 0.5) (layer F.Cu) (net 2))
 (segment (start 139.7 54.61) (end 137.16 57.15) (width 0.5) (layer F.Cu) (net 2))
 (segment (start 128.27 57.15) (end 127 55.88) (width 0.5) (layer F.Cu) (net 2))
 (segment (start 127 52.07) (end 130.81 48.26) (width 0.5) (layer F.Cu) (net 2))
 (segment (start 127 55.88) (end 127 52.07) (width 0.5) (layer F.Cu) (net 2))
 (segment (start 172.72 52.07) (end 175.26 54.61) (width 0.5) (layer F.Cu) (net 2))
 (segment (start 139.7 54.61) (end 142.24 52.07) (width 0.5) (layer F.Cu) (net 2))
 (segment (start 142.24 52.07) (end 172.72 52.07) (width 0.5) (layer F.Cu) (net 2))
 (segment (start 180.34 41.91) (end 180.34 44.45) (width 0.5) (layer F.Cu) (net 2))
 (segment (start 180.34 44.45) (end 172.72 52.07) (width 0.5) (layer F.Cu) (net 2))
 (segment (start 167.64 107.95) (end 168.91 106.68) (width 0.5) (layer F.Cu) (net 2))
 (segment (start 175.840002 106.68) (end 176.53 107.369998) (width 0.5) (layer F.Cu) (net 2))
 (segment (start 168.91 106.68) (end 175.840002 106.68) (width 0.5) (layer F.Cu) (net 2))
 (segment (start 176.53 108.530002) (end 174.570002 110.49) (width 0.5) (layer F.Cu) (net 2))
 (segment (start 176.53 107.369998) (end 176.53 108.530002) (width 0.5) (layer F.Cu) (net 2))
 (segment (start 174.570002 110.49) (end 127 110.49) (width 0.5) (layer F.Cu) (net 2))
 (segment (start 127 110.49) (end 116.84 100.33) (width 0.5) (layer F.Cu) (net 2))
 (segment (start 116.84 100.33) (end 116.84 85.09) (width 0.5) (layer F.Cu) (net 2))
 (segment (start 121.92 82.55) (end 119.38 82.55) (width 0.5) (layer F.Cu) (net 2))
 (segment (start 123.19 83.82) (end 121.92 82.55) (width 0.5) (layer F.Cu) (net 2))
 (segment (start 116.84 85.09) (end 119.38 82.55) (width 0.5) (layer F.Cu) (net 2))
 (segment (start 123.19 83.82) (end 123.19 85.09) (width 0.5) (layer F.Cu) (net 2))
 (segment (start 123.19 85.09) (end 120.65 87.63) (width 0.5) (layer F.Cu) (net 2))
 (segment (start 210.82 116.84) (end 203.2 116.84) (width 0.5) (layer F.Cu) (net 2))
 (segment (start 184.839998 116.84) (end 176.53 108.530002) (width 0.5) (layer F.Cu) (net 2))
 (segment (start 203.2 116.84) (end 184.839998 116.84) (width 0.5) (layer F.Cu) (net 2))
 (segment (start 128.27 76.2) (end 121.92 82.55) (width 0.5) (layer F.Cu) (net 2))
 (segment (start 128.27 57.15) (end 128.27 76.2) (width 0.5) (layer F.Cu) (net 2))
 (segment (start 130.790001 41.929999) (end 130.790001 48.240001) (width 0.5) (layer F.Cu) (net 2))
 (segment (start 130.790001 41.929999) (end 130.790001 42.470003) (width 0.5) (layer F.Cu) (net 2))
 (segment (start 130.790001 37.206357) (end 130.790001 41.929999) (width 0.5) (layer F.Cu) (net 2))
 (segment (start 172.72 41.91) (end 172.72 36.83) (width 1.4) (layer F.Cu) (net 6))
 (segment (start 175.26 41.91) (end 175.26 36.83) (width 1.4) (layer F.Cu) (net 7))
 (segment (start 177.8 36.83) (end 177.8 41.91) (width 1.4) (layer F.Cu) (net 8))
 (segment (start 142.24 36.83) (end 142.24 41.91) (width 1.4) (layer F.Cu) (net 12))
 (segment (start 139.7 36.83) (end 139.7 41.91) (width 1.4) (layer F.Cu) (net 11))
 (segment (start 137.16 36.83) (end 137.16 41.91) (width 1.4) (layer F.Cu) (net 10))
 (segment (start 134.62 36.83) (end 134.62 41.91) (width 1.4) (layer F.Cu) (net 9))
 (segment (start 175.26 62.23) (end 175.26 64.77) (width 0.25) (layer F.Cu) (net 31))
 (segment (start 174.134999 61.104999) (end 175.26 62.23) (width 0.25) (layer F.Cu) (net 31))
 (segment (start 144.78 54.61) (end 151.274999 61.104999) (width 0.25) (layer F.Cu) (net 31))
 (segment (start 151.274999 61.104999) (end 174.134999 61.104999) (width 0.25) (layer F.Cu) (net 31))
 (segment (start 177.8 62.23) (end 177.8 64.77) (width 0.25) (layer F.Cu) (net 32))
 (segment (start 176.224989 60.654989) (end 177.8 62.23) (width 0.25) (layer F.Cu) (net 32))
 (segment (start 147.32 54.61) (end 153.364989 60.654989) (width 0.25) (layer F.Cu) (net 32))
 (segment (start 153.364989 60.654989) (end 176.224989 60.654989) (width 0.25) (layer F.Cu) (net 32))
 (segment (start 203.2 82.55) (end 203.2 81.4364) (width 0.25) (layer F.Cu) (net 39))
 (segment (start 187.96 66.1964) (end 203.2 81.4364) (width 0.25) (layer F.Cu) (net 39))
 (segment (start 187.96 64.77) (end 187.96 66.1964) (width 0.25) (layer F.Cu) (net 39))
 (segment (start 209.55 53.34) (end 209.55 49.53) (width 0.25) (layer F.Cu) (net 37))
 (segment (start 194.31 53.34) (end 185.42 62.23) (width 0.25) (layer F.Cu) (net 37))
 (segment (start 209.55 53.34) (end 194.31 53.34) (width 0.25) (layer F.Cu) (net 37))
 (segment (start 185.42 62.23) (end 185.42 64.77) (width 0.25) (layer F.Cu) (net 37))
 (segment (start 187.96 36.83) (end 187.96 43.18) (width 0.25) (layer F.Cu) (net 17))
 (segment (start 168.91 64.77) (end 170.18 66.04) (width 0.25) (layer F.Cu) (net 17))
 (segment (start 180.735002 66.04) (end 181.754999 65.020003) (width 0.25) (layer F.Cu) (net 17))
 (segment (start 170.18 66.04) (end 180.735002 66.04) (width 0.25) (layer F.Cu) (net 17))
 (segment (start 181.754999 65.020003) (end 181.754999 50.944999) (width 0.25) (layer F.Cu) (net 17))
 (segment (start 187.96 44.739998) (end 187.96 36.83) (width 0.25) (layer F.Cu) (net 17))
 (segment (start 181.754999 50.944999) (end 187.96 44.739998) (width 0.25) (layer F.Cu) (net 17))
 (segment (start 180.34 107.95) (end 188.88 99.41) (width 0.25) (layer F.Cu) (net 13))
 (segment (start 207.01 99.06) (end 203.2 99.06) (width 0.25) (layer F.Cu) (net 13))
 (segment (start 189.23 99.06) (end 203.2 99.06) (width 0.25) (layer F.Cu) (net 13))
 (segment (start 180.34 107.95) (end 189.23 99.06) (width 0.25) (layer F.Cu) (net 13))
 (segment (start 133.35 97.79) (end 166.37 64.77) (width 0.25) (layer F.Cu) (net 27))
 (segment (start 120.65 97.79) (end 133.35 97.79) (width 0.25) (layer F.Cu) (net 27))
 (segment (start 203.2 101.6) (end 207.01 101.6) (width 0.25) (layer F.Cu) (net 14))
 (segment (start 189.23 101.6) (end 182.88 107.95) (width 0.25) (layer F.Cu) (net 14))
 (segment (start 203.2 101.6) (end 189.23 101.6) (width 0.25) (layer F.Cu) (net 14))
 (segment (start 135.89 92.71) (end 163.83 64.77) (width 0.25) (layer F.Cu) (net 26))
 (segment (start 120.65 92.71) (end 135.89 92.71) (width 0.25) (layer F.Cu) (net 26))
 (segment (start 207.01 104.14) (end 203.2 104.14) (width 0.25) (layer F.Cu) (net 15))
 (segment (start 189.23 104.14) (end 203.2 104.14) (width 0.25) (layer F.Cu) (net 15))
 (segment (start 185.42 107.95) (end 189.23 104.14) (width 0.25) (layer F.Cu) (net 15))
 (segment (start 154.69 71.12) (end 161.04 64.77) (width 0.25) (layer F.Cu) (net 25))
 (segment (start 135.64 90.17) (end 161.04 64.77) (width 0.25) (layer F.Cu) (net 25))
 (segment (start 120.65 90.17) (end 135.64 90.17) (width 0.25) (layer F.Cu) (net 25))
 (segment (start 203.2 106.68) (end 207.01 106.68) (width 0.25) (layer F.Cu) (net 16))
 (segment (start 189.23 106.68) (end 187.96 107.95) (width 0.25) (layer F.Cu) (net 16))
 (segment (start 203.2 106.68) (end 189.23 106.68) (width 0.25) (layer F.Cu) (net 16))
 (segment (start 157.700001 65.569999) (end 158.5 64.77) (width 0.25) (layer F.Cu) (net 24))
 (segment (start 134.464999 88.805001) (end 157.700001 65.569999) (width 0.25) (layer F.Cu) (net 24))
 (segment (start 120.275997 88.805001) (end 134.464999 88.805001) (width 0.25) (layer F.Cu) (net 24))
 (segment (start 119.474999 89.605999) (end 120.275997 88.805001) (width 0.25) (layer F.Cu) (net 24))
 (segment (start 119.474999 94.074999) (end 119.474999 89.605999) (width 0.25) (layer F.Cu) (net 24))
 (segment (start 120.65 95.25) (end 119.474999 94.074999) (width 0.25) (layer F.Cu) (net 24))
 (segment (start 154.94 37.37) (end 155.894594 37.37) (width 0.5) (layer F.Cu) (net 3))
 (segment (start 155.894594 37.37) (end 165.324594 27.94) (width 0.5) (layer F.Cu) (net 3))
 (segment (start 165.324594 27.94) (end 201.93 27.94) (width 0.5) (layer F.Cu) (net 3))
 (segment (start 201.93 27.94) (end 223.52 49.53) (width 0.5) (layer F.Cu) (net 3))
 (segment (start 202.336401 89.306401) (end 203.2 90.17) (width 0.5) (layer F.Cu) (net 3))
 (segment (start 201.886399 88.856399) (end 202.336401 89.306401) (width 0.5) (layer F.Cu) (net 3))
 (segment (start 201.886399 86.403601) (end 201.886399 88.856399) (width 0.5) (layer F.Cu) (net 3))
 (segment (start 203.2 85.09) (end 201.886399 86.403601) (width 0.5) (layer F.Cu) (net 3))
 (segment (start 223.52 49.53) (end 223.52 101.6) (width 0.5) (layer F.Cu) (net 3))
 (segment (start 223.52 101.6) (end 213.36 111.76) (width 0.5) (layer F.Cu) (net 3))
 (segment (start 213.36 111.76) (end 181.61 111.76) (width 0.5) (layer F.Cu) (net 3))
 (segment (start 179.089999 109.239999) (end 179.089999 104.159999) (width 0.5) (layer F.Cu) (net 3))
 (segment (start 181.61 111.76) (end 179.089999 109.239999) (width 0.5) (layer F.Cu) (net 3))
 (segment (start 179.089999 104.159999) (end 190.539998 92.71) (width 0.5) (layer F.Cu) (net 3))
 (segment (start 200.66 92.71) (end 203.2 90.17) (width 0.5) (layer F.Cu) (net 3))
 (segment (start 190.539998 92.71) (end 200.66 92.71) (width 0.5) (layer F.Cu) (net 3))
 (segment (start 217.17 52.07) (end 214.63 49.53) (width 0.25) (layer F.Cu) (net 46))
 (segment (start 205.74 90.17) (end 217.17 78.74) (width 0.25) (layer F.Cu) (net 46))
 (segment (start 217.17 78.74) (end 217.17 52.07) (width 0.25) (layer F.Cu) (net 46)))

